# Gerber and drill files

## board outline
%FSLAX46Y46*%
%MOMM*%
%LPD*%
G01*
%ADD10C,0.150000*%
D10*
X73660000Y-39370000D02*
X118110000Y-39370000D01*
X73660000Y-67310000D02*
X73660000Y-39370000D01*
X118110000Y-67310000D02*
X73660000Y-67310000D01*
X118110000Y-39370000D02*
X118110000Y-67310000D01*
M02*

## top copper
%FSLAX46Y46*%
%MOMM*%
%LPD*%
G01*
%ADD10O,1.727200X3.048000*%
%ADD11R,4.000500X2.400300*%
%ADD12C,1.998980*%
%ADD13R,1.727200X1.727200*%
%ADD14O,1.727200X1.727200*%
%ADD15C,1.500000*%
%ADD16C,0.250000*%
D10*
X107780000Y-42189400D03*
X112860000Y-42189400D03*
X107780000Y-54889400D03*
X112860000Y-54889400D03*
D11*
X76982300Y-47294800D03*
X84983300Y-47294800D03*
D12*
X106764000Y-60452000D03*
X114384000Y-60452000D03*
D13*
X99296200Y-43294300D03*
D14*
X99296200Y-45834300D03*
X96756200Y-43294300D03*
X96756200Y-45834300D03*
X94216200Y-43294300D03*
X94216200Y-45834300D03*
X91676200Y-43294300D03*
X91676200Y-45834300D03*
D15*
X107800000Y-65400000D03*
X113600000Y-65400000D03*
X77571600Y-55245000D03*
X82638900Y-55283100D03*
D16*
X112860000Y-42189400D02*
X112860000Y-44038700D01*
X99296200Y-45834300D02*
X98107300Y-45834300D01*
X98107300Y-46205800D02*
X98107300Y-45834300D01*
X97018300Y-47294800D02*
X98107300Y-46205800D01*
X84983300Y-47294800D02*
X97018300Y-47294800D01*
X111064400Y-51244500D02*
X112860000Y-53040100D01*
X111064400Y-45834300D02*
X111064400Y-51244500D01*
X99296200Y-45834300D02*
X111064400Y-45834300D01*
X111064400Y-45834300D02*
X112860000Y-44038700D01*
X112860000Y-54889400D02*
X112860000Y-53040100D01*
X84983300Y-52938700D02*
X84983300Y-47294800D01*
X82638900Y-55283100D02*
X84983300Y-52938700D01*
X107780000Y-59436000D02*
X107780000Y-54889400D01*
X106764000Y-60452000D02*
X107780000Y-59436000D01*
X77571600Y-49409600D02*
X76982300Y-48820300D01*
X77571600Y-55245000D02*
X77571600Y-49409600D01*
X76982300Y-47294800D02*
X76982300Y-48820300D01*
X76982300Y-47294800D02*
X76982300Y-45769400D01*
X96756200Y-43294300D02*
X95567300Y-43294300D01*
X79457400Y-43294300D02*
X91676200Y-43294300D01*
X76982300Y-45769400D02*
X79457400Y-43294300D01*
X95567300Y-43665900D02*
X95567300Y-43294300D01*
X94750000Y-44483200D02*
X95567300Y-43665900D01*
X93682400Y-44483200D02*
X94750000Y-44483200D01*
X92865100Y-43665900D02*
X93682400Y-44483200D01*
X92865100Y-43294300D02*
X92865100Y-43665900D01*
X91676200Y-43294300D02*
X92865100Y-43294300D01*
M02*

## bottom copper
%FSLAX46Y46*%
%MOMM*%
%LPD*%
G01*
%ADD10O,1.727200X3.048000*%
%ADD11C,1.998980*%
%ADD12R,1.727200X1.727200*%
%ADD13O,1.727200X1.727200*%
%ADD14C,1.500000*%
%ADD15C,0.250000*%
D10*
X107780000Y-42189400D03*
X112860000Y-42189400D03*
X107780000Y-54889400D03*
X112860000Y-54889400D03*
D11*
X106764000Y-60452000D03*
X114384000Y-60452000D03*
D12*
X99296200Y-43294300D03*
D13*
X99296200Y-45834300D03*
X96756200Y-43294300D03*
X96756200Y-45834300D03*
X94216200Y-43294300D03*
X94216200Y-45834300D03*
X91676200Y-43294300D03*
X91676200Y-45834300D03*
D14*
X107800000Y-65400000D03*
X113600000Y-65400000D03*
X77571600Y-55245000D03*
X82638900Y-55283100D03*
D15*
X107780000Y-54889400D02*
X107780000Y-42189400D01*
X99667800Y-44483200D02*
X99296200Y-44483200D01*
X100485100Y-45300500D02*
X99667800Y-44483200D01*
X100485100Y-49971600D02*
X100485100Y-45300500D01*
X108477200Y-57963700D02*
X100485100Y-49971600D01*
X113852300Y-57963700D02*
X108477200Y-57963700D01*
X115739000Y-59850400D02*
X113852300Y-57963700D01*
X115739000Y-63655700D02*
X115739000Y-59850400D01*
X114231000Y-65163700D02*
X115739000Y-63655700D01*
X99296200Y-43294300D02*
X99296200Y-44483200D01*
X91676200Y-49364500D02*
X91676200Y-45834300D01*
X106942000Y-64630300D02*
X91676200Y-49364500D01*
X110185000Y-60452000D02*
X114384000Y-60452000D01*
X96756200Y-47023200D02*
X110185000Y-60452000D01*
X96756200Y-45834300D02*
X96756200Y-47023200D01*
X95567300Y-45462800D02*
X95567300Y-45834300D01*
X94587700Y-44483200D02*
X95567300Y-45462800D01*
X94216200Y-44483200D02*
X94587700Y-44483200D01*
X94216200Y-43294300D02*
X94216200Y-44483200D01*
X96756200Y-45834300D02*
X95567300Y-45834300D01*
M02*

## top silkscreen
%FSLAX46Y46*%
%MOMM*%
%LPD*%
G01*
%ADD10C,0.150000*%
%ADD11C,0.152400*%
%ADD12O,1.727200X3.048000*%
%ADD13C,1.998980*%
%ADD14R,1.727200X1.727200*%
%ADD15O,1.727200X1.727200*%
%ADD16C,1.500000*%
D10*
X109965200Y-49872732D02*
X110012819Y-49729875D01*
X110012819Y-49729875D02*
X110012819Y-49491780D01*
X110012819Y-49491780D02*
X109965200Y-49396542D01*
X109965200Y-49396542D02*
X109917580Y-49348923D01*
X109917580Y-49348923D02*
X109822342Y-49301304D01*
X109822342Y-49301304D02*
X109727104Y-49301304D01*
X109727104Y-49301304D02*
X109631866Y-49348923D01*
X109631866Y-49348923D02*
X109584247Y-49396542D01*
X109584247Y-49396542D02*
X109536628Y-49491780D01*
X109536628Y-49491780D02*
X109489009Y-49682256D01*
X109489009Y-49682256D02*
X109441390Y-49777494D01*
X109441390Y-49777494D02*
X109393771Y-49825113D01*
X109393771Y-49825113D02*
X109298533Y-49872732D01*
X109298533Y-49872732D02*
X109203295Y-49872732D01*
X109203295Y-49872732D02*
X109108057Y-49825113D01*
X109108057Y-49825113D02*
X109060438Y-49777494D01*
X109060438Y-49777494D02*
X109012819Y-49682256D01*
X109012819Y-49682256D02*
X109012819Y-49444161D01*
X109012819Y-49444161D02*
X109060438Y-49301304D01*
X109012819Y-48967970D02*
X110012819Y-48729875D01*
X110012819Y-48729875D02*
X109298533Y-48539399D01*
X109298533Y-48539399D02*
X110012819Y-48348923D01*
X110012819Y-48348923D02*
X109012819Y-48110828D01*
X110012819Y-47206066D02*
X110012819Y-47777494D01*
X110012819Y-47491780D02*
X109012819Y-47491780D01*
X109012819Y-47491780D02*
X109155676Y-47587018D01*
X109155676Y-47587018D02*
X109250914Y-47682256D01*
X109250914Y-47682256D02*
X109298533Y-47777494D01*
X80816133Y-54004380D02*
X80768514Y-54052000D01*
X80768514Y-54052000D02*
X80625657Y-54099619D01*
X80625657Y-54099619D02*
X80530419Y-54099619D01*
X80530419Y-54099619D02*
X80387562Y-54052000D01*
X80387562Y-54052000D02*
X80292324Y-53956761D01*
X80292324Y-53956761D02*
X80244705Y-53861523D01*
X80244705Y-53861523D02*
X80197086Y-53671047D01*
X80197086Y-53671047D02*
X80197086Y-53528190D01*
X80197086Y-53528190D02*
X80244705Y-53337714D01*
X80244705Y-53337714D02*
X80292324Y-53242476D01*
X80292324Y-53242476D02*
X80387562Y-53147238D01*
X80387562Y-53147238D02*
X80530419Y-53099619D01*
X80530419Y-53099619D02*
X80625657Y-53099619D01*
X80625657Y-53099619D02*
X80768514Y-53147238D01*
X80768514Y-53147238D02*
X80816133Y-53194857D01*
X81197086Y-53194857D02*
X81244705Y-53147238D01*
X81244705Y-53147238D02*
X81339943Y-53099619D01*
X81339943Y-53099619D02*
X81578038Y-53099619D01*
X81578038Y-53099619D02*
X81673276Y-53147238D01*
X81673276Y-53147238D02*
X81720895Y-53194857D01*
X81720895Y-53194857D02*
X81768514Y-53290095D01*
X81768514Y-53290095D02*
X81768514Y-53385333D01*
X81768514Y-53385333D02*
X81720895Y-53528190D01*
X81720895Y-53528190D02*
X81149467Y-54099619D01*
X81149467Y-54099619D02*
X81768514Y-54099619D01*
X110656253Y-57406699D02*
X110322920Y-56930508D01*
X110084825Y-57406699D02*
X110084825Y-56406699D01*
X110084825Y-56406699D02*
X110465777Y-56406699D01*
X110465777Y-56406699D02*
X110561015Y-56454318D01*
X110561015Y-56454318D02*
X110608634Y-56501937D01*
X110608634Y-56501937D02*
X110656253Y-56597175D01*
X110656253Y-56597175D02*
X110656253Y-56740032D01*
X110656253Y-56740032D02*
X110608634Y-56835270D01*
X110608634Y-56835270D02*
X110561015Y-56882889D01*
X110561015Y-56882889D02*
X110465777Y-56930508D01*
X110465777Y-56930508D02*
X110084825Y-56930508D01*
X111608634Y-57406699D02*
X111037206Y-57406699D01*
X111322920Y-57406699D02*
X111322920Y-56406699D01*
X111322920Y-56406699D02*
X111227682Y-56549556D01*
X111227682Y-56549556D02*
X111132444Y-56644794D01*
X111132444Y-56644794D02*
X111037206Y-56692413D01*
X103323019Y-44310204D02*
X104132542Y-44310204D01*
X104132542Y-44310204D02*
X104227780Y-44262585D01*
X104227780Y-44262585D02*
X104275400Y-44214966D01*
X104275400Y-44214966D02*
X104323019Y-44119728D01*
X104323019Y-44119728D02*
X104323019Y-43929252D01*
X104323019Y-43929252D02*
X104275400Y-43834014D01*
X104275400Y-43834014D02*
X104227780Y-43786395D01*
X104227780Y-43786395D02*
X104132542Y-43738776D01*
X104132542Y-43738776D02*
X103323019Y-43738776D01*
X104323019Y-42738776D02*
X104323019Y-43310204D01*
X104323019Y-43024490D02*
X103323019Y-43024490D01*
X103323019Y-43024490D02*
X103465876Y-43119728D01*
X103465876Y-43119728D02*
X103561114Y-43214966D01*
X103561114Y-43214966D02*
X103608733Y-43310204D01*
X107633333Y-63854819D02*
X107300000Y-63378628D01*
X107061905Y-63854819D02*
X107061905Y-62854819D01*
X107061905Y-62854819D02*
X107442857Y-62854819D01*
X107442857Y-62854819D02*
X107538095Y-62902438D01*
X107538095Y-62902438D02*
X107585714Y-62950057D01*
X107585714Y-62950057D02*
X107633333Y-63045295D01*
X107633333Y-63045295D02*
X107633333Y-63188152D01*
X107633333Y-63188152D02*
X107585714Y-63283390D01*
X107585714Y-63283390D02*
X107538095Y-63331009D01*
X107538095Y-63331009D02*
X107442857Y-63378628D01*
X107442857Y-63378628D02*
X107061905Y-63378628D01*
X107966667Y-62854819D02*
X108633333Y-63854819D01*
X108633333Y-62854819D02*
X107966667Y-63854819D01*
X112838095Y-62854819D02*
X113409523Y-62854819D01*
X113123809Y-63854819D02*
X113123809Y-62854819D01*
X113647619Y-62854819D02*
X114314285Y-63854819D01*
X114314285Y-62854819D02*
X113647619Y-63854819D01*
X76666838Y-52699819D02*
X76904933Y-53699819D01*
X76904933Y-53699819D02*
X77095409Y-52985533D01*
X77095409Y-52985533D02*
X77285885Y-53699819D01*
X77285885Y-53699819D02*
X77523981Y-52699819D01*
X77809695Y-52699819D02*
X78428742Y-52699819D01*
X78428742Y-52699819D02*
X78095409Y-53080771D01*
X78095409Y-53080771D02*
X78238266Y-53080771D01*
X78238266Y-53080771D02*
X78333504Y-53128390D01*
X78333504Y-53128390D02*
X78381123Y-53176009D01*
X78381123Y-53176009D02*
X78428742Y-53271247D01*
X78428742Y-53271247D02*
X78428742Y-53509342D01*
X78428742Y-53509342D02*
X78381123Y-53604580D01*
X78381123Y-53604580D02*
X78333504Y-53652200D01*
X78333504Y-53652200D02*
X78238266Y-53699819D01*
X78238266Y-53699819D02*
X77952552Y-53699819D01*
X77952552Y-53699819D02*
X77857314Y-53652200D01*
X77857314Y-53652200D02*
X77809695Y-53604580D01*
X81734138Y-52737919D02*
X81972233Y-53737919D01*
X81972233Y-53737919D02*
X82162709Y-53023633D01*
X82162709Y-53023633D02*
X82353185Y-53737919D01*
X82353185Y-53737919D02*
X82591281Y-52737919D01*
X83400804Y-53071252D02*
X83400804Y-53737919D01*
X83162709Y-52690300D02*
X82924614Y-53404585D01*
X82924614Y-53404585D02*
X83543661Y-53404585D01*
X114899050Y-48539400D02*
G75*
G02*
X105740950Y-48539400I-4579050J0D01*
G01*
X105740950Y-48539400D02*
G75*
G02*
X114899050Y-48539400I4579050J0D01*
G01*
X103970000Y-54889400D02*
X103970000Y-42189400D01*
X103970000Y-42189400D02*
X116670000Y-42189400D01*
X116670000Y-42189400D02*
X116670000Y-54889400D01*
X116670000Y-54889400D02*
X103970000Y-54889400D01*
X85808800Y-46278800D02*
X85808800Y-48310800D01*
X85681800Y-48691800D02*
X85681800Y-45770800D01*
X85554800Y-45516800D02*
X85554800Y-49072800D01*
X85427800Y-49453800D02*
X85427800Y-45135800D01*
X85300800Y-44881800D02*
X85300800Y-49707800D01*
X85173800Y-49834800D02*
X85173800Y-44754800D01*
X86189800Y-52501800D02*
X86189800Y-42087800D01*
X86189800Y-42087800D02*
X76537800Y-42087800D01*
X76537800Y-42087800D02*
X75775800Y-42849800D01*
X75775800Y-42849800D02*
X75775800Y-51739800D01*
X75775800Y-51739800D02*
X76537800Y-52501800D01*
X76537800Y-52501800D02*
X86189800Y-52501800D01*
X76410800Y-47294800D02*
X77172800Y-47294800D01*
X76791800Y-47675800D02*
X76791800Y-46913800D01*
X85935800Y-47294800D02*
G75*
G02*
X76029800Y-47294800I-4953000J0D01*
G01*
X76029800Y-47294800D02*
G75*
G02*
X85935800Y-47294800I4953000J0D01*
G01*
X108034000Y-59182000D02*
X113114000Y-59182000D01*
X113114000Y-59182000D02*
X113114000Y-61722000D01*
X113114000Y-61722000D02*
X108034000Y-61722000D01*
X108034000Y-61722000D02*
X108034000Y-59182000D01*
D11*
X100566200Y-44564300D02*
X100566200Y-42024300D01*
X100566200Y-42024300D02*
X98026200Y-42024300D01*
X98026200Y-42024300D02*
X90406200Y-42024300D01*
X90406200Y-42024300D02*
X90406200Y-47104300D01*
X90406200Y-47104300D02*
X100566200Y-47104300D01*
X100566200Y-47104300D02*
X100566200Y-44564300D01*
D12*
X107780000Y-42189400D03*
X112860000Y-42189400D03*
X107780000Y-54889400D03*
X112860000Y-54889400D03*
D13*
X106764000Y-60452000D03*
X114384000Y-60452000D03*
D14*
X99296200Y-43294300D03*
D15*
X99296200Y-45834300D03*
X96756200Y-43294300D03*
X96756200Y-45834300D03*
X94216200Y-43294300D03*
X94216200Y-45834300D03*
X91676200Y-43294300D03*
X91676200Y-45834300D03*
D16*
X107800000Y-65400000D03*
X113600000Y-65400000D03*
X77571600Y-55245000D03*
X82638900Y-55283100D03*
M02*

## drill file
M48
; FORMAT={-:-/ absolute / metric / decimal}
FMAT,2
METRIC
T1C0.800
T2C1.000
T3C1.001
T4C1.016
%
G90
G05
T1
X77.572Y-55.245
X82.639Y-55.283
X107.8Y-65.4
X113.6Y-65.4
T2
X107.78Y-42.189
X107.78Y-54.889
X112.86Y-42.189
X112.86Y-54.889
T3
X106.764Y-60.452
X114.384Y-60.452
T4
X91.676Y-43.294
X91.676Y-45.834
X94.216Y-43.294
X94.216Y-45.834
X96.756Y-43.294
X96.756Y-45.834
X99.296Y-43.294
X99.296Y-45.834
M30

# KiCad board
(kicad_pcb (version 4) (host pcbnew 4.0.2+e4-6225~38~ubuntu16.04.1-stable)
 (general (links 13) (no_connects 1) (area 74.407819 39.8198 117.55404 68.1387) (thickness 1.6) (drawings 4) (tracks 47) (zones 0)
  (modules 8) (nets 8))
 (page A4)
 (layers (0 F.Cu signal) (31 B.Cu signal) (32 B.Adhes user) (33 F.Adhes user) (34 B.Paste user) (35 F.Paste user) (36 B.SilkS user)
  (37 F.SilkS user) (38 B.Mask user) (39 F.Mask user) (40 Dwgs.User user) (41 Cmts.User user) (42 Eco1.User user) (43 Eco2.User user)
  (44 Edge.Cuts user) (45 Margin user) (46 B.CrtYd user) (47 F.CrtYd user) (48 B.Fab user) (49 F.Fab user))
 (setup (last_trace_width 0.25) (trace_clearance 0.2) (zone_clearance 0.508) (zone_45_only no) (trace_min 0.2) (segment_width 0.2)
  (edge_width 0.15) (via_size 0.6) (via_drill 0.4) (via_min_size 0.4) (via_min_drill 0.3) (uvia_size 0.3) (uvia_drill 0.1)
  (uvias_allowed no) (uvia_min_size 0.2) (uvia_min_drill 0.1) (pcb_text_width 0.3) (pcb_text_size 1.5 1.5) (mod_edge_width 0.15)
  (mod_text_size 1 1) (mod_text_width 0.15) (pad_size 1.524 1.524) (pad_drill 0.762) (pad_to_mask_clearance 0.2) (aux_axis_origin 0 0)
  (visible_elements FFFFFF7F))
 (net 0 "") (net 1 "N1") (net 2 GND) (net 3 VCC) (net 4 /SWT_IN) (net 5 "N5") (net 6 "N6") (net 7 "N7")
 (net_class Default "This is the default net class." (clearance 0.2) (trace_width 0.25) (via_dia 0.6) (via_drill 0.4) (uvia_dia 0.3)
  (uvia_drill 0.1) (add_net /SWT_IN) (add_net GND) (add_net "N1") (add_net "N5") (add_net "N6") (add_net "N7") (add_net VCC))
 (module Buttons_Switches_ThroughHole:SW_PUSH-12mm (layer F.Cu) (at 110.32 48.5394 90)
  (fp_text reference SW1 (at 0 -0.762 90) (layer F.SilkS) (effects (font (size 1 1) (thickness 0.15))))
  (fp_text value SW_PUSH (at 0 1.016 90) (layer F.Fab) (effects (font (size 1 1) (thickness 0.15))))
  (fp_circle (center 0 0) (end 3.81 2.54) (layer F.SilkS) (width 0.15))
  (fp_line (start -6.35 -6.35) (end 6.35 -6.35) (layer F.SilkS) (width 0.15))
  (fp_line (start 6.35 -6.35) (end 6.35 6.35) (layer F.SilkS) (width 0.15))
  (fp_line (start 6.35 6.35) (end -6.35 6.35) (layer F.SilkS) (width 0.15))
  (fp_line (start -6.35 6.35) (end -6.35 -6.35) (layer F.SilkS) (width 0.15))
  (pad 1 thru_hole oval (at 6.35 -2.54 90) (size 3.048 1.7272) (drill 1) (layers *.Cu *.Mask F.SilkS) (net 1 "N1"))
  (pad 2 thru_hole oval (at 6.35 2.54 90) (size 3.048 1.7272) (drill 1) (layers *.Cu *.Mask F.SilkS) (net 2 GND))
  (pad 1 thru_hole oval (at -6.35 -2.54 90) (size 3.048 1.7272) (drill 1) (layers *.Cu *.Mask F.SilkS) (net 1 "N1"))
  (pad 2 thru_hole oval (at -6.35 2.54 90) (size 3.048 1.7272) (drill 1) (layers *.Cu *.Mask F.SilkS) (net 2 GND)))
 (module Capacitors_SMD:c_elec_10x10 (layer F.Cu) (at 80.9828 47.2948 180)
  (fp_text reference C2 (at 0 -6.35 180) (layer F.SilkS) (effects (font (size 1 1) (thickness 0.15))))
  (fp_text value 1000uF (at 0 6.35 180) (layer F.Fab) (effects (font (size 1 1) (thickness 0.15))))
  (fp_line (start -4.826 1.016) (end -4.826 -1.016) (layer F.SilkS) (width 0.15))
  (fp_line (start -4.699 -1.397) (end -4.699 1.524) (layer F.SilkS) (width 0.15))
  (fp_line (start -4.572 1.778) (end -4.572 -1.778) (layer F.SilkS) (width 0.15))
  (fp_line (start -4.445 -2.159) (end -4.445 2.159) (layer F.SilkS) (width 0.15))
  (fp_line (start -4.318 2.413) (end -4.318 -2.413) (layer F.SilkS) (width 0.15))
  (fp_line (start -4.191 -2.54) (end -4.191 2.54) (layer F.SilkS) (width 0.15))
  (fp_line (start -5.207 -5.207) (end -5.207 5.207) (layer F.SilkS) (width 0.15))
  (fp_line (start -5.207 5.207) (end 4.445 5.207) (layer F.SilkS) (width 0.15))
  (fp_line (start 4.445 5.207) (end 5.207 4.445) (layer F.SilkS) (width 0.15))
  (fp_line (start 5.207 4.445) (end 5.207 -4.445) (layer F.SilkS) (width 0.15))
  (fp_line (start 5.207 -4.445) (end 4.445 -5.207) (layer F.SilkS) (width 0.15))
  (fp_line (start 4.445 -5.207) (end -5.207 -5.207) (layer F.SilkS) (width 0.15))
  (fp_line (start 4.572 0) (end 3.81 0) (layer F.SilkS) (width 0.15))
  (fp_line (start 4.191 -0.381) (end 4.191 0.381) (layer F.SilkS) (width 0.15))
  (fp_circle (center 0 0) (end 4.953 0) (layer F.SilkS) (width 0.15))
  (pad 1 smd rect (at 4.0005 0 180) (size 4.0005 2.4003) (layers F.Cu F.Paste F.Mask) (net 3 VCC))
  (pad 2 smd rect (at -4.0005 0 180) (size 4.0005 2.4003) (layers F.Cu F.Paste F.Mask) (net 2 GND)))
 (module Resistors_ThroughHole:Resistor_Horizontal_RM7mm (layer F.Cu) (at 106.764 60.452)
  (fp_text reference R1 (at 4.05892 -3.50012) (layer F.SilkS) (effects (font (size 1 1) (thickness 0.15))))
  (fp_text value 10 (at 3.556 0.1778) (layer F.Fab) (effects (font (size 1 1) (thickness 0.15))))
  (fp_line (start 1.27 -1.27) (end 6.35 -1.27) (layer F.SilkS) (width 0.15))
  (fp_line (start 6.35 -1.27) (end 6.35 1.27) (layer F.SilkS) (width 0.15))
  (fp_line (start 6.35 1.27) (end 1.27 1.27) (layer F.SilkS) (width 0.15))
  (fp_line (start 1.27 1.27) (end 1.27 -1.27) (layer F.SilkS) (width 0.15))
  (pad 1 thru_hole circle (at 0 0) (size 1.99898 1.99898) (drill 1.00076) (layers *.Cu *.SilkS *.Mask) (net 1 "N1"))
  (pad 2 thru_hole circle (at 7.62 0) (size 1.99898 1.99898) (drill 1.00076) (layers *.Cu *.SilkS *.Mask) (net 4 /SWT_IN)))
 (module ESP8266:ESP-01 (layer F.Cu) (at 99.2962 43.2943 270)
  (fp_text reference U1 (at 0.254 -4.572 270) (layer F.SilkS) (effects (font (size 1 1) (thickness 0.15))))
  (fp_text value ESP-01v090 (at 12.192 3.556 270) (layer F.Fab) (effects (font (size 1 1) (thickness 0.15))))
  (fp_line (start 1.27 -1.27) (end -1.27 -1.27) (layer F.SilkS) (width 0.1524))
  (fp_line (start -1.27 -1.27) (end -1.27 1.27) (layer F.SilkS) (width 0.1524))
  (fp_line (start -1.27 1.27) (end -1.27 8.89) (layer F.SilkS) (width 0.1524))
  (fp_line (start -1.27 8.89) (end 3.81 8.89) (layer F.SilkS) (width 0.1524))
  (fp_line (start 3.81 8.89) (end 3.81 -1.27) (layer F.SilkS) (width 0.1524))
  (fp_line (start 3.81 -1.27) (end 1.27 -1.27) (layer F.SilkS) (width 0.1524))
  (pad 1 thru_hole rect (at 0 0 270) (size 1.7272 1.7272) (drill 1.016) (layers *.Cu *.Mask F.SilkS) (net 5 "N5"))
  (pad 2 thru_hole oval (at 2.54 0 270) (size 1.7272 1.7272) (drill 1.016) (layers *.Cu *.Mask F.SilkS) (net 2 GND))
  (pad 3 thru_hole oval (at 0 2.54 270) (size 1.7272 1.7272) (drill 1.016) (layers *.Cu *.Mask F.SilkS) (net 3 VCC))
  (pad 4 thru_hole oval (at 2.54 2.54 270) (size 1.7272 1.7272) (drill 1.016) (layers *.Cu *.Mask F.SilkS) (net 4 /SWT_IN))
  (pad 5 thru_hole oval (at 0 5.08 270) (size 1.7272 1.7272) (drill 1.016) (layers *.Cu *.Mask F.SilkS) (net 4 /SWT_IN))
  (pad 6 thru_hole oval (at 2.54 5.08 270) (size 1.7272 1.7272) (drill 1.016) (layers *.Cu *.Mask F.SilkS) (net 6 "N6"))
  (pad 7 thru_hole oval (at 0 7.62 270) (size 1.7272 1.7272) (drill 1.016) (layers *.Cu *.Mask F.SilkS) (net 3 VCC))
  (pad 8 thru_hole oval (at 2.54 7.62 270) (size 1.7272 1.7272) (drill 1.016) (layers *.Cu *.Mask F.SilkS) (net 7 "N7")))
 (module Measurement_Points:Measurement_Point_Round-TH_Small (layer F.Cu) (at 107.8 65.4)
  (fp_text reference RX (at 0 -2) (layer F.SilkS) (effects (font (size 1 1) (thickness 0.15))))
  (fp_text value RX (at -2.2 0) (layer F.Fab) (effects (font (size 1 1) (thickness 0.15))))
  (pad 1 thru_hole circle (at 0 0) (size 1.5 1.5) (drill 0.8) (layers *.Cu *.Mask F.SilkS) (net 7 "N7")))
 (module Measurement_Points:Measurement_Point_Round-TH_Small (layer F.Cu) (at 113.6 65.4)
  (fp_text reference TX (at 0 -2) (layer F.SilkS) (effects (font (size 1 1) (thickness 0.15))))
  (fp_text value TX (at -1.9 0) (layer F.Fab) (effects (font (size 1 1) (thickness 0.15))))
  (pad 1 thru_hole circle (at 0 0) (size 1.5 1.5) (drill 0.8) (layers *.Cu *.Mask F.SilkS) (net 5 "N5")))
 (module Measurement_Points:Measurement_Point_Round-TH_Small (layer F.Cu) (at 77.5716 55.245)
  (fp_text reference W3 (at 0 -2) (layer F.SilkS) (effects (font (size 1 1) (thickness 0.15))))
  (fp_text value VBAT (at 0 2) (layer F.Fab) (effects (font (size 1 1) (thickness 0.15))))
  (pad 1 thru_hole circle (at 0 0) (size 1.5 1.5) (drill 0.8) (layers *.Cu *.Mask F.SilkS) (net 3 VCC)))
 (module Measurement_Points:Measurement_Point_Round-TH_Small (layer F.Cu) (at 82.6389 55.2831)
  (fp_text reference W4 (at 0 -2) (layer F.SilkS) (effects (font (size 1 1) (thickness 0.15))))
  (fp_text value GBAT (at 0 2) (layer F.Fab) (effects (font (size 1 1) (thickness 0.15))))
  (pad 1 thru_hole circle (at 0 0) (size 1.5 1.5) (drill 0.8) (layers *.Cu *.Mask F.SilkS) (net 2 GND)))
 (gr_line (start 73.66 39.37) (end 118.11 39.37) (angle 90) (layer Edge.Cuts) (width 0.15))
 (gr_line (start 73.66 67.31) (end 73.66 39.37) (angle 90) (layer Edge.Cuts) (width 0.15))
 (gr_line (start 118.11 67.31) (end 73.66 67.31) (angle 90) (layer Edge.Cuts) (width 0.15))
 (gr_line (start 118.11 39.37) (end 118.11 67.31) (angle 90) (layer Edge.Cuts) (width 0.15))
 (segment (start 112.86 42.1894) (end 112.86 44.0387) (width 0.25) (layer F.Cu) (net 2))
 (segment (start 99.2962 45.8343) (end 98.1073 45.8343) (width 0.25) (layer F.Cu) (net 2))
 (segment (start 98.1073 46.2058) (end 98.1073 45.8343) (width 0.25) (layer F.Cu) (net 2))
 (segment (start 97.0183 47.2948) (end 98.1073 46.2058) (width 0.25) (layer F.Cu) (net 2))
 (segment (start 84.9833 47.2948) (end 97.0183 47.2948) (width 0.25) (layer F.Cu) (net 2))
 (segment (start 111.0644 51.2445) (end 112.86 53.0401) (width 0.25) (layer F.Cu) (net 2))
 (segment (start 111.0644 45.8343) (end 111.0644 51.2445) (width 0.25) (layer F.Cu) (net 2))
 (segment (start 99.2962 45.8343) (end 111.0644 45.8343) (width 0.25) (layer F.Cu) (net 2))
 (segment (start 111.0644 45.8343) (end 112.86 44.0387) (width 0.25) (layer F.Cu) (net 2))
 (segment (start 112.86 54.8894) (end 112.86 53.0401) (width 0.25) (layer F.Cu) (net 2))
 (segment (start 84.9833 52.9387) (end 84.9833 47.2948) (width 0.25) (layer F.Cu) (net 2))
 (segment (start 82.6389 55.2831) (end 84.9833 52.9387) (width 0.25) (layer F.Cu) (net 2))
 (segment (start 107.78 59.436) (end 107.78 54.8894) (width 0.25) (layer F.Cu) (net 1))
 (segment (start 106.764 60.452) (end 107.78 59.436) (width 0.25) (layer F.Cu) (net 1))
 (segment (start 107.78 54.8894) (end 107.78 42.1894) (width 0.25) (layer B.Cu) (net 1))
 (segment (start 99.6678 44.4832) (end 99.2962 44.4832) (width 0.25) (layer B.Cu) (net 5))
 (segment (start 100.4851 45.3005) (end 99.6678 44.4832) (width 0.25) (layer B.Cu) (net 5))
 (segment (start 100.4851 49.9716) (end 100.4851 45.3005) (width 0.25) (layer B.Cu) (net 5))
 (segment (start 108.4772 57.9637) (end 100.4851 49.9716) (width 0.25) (layer B.Cu) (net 5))
 (segment (start 113.8523 57.9637) (end 108.4772 57.9637) (width 0.25) (layer B.Cu) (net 5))
 (segment (start 115.739 59.8504) (end 113.8523 57.9637) (width 0.25) (layer B.Cu) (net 5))
 (segment (start 115.739 63.6557) (end 115.739 59.8504) (width 0.25) (layer B.Cu) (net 5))
 (segment (start 114.231 65.1637) (end 115.739 63.6557) (width 0.25) (layer B.Cu) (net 5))
 (segment (start 99.2962 43.2943) (end 99.2962 44.4832) (width 0.25) (layer B.Cu) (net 5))
 (segment (start 91.6762 49.3645) (end 91.6762 45.8343) (width 0.25) (layer B.Cu) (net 7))
 (segment (start 106.942 64.6303) (end 91.6762 49.3645) (width 0.25) (layer B.Cu) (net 7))
 (segment (start 77.5716 49.4096) (end 76.9823 48.8203) (width 0.25) (layer F.Cu) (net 3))
 (segment (start 77.5716 55.245) (end 77.5716 49.4096) (width 0.25) (layer F.Cu) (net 3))
 (segment (start 76.9823 47.2948) (end 76.9823 48.8203) (width 0.25) (layer F.Cu) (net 3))
 (segment (start 76.9823 47.2948) (end 76.9823 45.7694) (width 0.25) (layer F.Cu) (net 3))
 (segment (start 96.7562 43.2943) (end 95.5673 43.2943) (width 0.25) (layer F.Cu) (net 3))
 (segment (start 79.4574 43.2943) (end 91.6762 43.2943) (width 0.25) (layer F.Cu) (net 3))
 (segment (start 76.9823 45.7694) (end 79.4574 43.2943) (width 0.25) (layer F.Cu) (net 3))
 (segment (start 95.5673 43.6659) (end 95.5673 43.2943) (width 0.25) (layer F.Cu) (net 3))
 (segment (start 94.75 44.4832) (end 95.5673 43.6659) (width 0.25) (layer F.Cu) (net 3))
 (segment (start 93.6824 44.4832) (end 94.75 44.4832) (width 0.25) (layer F.Cu) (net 3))
 (segment (start 92.8651 43.6659) (end 93.6824 44.4832) (width 0.25) (layer F.Cu) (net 3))
 (segment (start 92.8651 43.2943) (end 92.8651 43.6659) (width 0.25) (layer F.Cu) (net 3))
 (segment (start 91.6762 43.2943) (end 92.8651 43.2943) (width 0.25) (layer F.Cu) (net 3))
 (segment (start 110.185 60.452) (end 114.384 60.452) (width 0.25) (layer B.Cu) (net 4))
 (segment (start 96.7562 47.0232) (end 110.185 60.452) (width 0.25) (layer B.Cu) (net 4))
 (segment (start 96.7562 45.8343) (end 96.7562 47.0232) (width 0.25) (layer B.Cu) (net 4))
 (segment (start 95.5673 45.4628) (end 95.5673 45.8343) (width 0.25) (layer B.Cu) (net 4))
 (segment (start 94.5877 44.4832) (end 95.5673 45.4628) (width 0.25) (layer B.Cu) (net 4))
 (segment (start 94.2162 44.4832) (end 94.5877 44.4832) (width 0.25) (layer B.Cu) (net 4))
 (segment (start 94.2162 43.2943) (end 94.2162 44.4832) (width 0.25) (layer B.Cu) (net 4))
 (segment (start 96.7562 45.8343) (end 95.5673 45.8343) (width 0.25) (layer B.Cu) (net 4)))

